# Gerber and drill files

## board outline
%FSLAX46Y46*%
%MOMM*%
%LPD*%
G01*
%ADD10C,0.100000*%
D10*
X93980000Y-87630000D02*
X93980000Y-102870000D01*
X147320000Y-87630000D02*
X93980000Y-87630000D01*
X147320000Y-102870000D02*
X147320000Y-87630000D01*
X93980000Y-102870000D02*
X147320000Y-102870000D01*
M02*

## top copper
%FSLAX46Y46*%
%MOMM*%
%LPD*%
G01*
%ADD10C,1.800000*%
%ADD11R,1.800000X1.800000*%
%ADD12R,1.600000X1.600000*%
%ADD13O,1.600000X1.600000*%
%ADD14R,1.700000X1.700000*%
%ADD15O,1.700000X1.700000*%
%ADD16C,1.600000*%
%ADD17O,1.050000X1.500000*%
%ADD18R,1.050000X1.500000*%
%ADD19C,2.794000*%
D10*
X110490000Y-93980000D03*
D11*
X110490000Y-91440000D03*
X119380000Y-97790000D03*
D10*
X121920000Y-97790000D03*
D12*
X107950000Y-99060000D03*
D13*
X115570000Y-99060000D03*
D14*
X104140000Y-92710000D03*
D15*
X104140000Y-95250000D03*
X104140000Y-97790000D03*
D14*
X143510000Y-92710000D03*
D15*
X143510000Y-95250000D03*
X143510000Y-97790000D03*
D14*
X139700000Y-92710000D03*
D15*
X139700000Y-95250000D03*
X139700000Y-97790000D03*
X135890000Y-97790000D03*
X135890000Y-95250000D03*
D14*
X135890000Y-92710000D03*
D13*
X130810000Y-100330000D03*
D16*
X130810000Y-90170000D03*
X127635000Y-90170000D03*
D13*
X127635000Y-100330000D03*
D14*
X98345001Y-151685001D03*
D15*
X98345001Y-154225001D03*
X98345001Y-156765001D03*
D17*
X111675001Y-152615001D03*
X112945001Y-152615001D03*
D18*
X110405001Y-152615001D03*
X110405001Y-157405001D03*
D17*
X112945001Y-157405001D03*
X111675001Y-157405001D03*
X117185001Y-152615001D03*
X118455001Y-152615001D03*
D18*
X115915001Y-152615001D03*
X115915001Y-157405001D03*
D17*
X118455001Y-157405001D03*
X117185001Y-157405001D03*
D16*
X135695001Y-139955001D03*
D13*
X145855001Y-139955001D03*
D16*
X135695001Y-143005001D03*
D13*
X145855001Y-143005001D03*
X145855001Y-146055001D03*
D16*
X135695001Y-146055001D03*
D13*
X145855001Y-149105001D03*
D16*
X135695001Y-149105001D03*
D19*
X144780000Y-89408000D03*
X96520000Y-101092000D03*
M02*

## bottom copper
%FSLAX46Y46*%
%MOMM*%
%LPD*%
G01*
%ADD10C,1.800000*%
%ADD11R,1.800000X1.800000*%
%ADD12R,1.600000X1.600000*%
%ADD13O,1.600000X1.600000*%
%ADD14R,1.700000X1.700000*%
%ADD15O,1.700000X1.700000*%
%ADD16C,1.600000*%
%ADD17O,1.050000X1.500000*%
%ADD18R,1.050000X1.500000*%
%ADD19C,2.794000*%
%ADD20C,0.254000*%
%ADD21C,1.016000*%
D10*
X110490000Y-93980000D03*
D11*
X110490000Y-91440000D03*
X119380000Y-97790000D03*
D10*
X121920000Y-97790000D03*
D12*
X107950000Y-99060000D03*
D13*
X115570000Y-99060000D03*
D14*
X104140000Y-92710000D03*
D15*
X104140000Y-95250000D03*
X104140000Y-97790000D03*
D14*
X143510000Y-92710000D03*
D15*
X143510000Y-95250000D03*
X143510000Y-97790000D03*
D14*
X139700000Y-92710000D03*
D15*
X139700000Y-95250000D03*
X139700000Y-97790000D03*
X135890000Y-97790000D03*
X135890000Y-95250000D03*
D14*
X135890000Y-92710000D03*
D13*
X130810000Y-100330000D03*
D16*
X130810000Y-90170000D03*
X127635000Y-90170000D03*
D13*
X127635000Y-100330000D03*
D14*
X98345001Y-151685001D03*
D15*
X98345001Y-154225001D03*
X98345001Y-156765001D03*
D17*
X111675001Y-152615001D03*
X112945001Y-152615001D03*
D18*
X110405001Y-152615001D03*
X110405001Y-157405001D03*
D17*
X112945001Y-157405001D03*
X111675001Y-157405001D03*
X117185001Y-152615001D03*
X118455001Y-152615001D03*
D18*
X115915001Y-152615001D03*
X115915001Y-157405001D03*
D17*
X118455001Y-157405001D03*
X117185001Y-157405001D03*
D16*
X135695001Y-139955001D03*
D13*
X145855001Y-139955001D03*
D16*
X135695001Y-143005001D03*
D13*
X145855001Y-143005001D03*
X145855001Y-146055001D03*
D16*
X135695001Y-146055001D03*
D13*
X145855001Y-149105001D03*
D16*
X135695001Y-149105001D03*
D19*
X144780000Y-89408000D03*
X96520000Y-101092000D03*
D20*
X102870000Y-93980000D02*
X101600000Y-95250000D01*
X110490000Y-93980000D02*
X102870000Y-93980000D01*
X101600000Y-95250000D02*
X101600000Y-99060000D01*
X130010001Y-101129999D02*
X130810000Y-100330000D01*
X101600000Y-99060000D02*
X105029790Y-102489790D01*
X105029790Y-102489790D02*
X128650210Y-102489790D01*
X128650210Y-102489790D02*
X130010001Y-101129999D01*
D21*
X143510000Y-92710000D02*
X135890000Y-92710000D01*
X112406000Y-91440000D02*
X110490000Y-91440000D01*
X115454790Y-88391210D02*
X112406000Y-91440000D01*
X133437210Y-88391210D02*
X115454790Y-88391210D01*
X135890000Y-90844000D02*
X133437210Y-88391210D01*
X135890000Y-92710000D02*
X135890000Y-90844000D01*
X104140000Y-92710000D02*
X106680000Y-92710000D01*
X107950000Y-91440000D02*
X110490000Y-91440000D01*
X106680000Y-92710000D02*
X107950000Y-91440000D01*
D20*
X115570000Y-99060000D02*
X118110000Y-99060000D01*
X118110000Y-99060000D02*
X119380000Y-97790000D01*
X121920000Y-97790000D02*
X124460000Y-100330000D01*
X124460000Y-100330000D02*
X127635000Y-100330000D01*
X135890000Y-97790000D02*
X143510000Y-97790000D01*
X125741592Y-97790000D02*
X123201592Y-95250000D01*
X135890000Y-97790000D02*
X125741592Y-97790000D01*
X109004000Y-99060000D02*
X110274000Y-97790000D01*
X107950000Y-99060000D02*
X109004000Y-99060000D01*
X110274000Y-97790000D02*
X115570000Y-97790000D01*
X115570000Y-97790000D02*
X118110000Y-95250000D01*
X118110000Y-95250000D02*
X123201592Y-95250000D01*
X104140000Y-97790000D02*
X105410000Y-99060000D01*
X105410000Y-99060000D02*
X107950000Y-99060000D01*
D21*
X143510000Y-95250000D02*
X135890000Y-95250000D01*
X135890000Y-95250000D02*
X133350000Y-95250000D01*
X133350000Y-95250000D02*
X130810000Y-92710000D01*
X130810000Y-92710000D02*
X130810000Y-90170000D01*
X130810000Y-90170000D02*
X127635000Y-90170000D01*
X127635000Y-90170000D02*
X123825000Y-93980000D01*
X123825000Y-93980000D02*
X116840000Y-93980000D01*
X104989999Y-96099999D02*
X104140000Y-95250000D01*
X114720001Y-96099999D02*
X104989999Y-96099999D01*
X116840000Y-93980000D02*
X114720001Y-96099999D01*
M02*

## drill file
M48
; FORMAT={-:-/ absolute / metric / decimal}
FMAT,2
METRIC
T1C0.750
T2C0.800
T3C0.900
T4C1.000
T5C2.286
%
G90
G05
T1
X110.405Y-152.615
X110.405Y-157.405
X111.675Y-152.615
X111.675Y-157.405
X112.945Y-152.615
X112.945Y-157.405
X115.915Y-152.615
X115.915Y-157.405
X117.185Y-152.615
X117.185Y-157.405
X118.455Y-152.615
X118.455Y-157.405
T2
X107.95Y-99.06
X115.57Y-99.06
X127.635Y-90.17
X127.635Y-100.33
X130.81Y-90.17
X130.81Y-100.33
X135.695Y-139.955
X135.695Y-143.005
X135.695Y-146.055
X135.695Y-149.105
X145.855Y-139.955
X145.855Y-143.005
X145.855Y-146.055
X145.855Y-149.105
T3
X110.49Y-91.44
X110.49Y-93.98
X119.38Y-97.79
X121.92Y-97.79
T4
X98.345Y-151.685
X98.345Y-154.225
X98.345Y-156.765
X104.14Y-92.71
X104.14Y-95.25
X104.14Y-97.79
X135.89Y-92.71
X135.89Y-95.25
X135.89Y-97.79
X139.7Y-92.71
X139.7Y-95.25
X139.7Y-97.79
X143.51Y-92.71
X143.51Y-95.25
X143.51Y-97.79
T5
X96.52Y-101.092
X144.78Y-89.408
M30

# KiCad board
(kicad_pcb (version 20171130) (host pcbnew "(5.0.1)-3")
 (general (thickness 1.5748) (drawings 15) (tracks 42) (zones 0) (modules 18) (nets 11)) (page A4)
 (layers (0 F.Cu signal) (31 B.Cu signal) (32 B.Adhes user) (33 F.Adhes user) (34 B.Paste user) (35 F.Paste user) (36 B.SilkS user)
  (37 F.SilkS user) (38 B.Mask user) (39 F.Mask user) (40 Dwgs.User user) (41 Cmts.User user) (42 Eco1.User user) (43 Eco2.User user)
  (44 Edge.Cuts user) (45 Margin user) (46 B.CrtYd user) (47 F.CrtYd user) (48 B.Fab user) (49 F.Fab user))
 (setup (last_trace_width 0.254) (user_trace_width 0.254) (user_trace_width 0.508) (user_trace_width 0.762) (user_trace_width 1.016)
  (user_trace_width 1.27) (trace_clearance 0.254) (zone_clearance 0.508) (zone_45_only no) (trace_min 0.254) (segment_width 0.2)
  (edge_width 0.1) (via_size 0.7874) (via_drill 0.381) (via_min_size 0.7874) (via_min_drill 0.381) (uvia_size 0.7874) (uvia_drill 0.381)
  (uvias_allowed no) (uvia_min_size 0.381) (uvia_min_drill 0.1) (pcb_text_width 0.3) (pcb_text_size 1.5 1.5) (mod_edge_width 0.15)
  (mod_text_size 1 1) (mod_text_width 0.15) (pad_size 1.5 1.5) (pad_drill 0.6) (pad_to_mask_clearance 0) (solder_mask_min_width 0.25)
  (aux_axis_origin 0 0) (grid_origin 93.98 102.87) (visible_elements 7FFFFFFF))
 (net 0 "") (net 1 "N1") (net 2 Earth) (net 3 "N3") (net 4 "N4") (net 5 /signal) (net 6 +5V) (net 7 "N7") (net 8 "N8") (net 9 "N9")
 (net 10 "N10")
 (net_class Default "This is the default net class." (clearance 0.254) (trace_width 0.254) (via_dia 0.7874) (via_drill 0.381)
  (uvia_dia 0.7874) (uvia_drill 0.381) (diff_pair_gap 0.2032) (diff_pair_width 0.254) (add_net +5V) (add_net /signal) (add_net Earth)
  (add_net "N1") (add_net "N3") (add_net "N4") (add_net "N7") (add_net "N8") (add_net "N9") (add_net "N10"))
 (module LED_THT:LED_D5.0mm (layer F.Cu) (at 110.49 91.44 270)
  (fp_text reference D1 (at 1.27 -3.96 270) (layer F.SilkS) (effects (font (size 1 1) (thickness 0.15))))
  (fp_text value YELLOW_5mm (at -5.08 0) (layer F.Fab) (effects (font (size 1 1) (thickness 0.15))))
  (pad 2 thru_hole circle (at 2.54 0 270) (size 1.8 1.8) (drill 0.9) (layers *.Cu *.Mask) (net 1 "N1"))
  (pad 1 thru_hole rect (at 0 0 270) (size 1.8 1.8) (drill 0.9) (layers *.Cu *.Mask) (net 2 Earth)))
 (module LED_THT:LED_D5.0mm (layer F.Cu) (at 119.38 97.79)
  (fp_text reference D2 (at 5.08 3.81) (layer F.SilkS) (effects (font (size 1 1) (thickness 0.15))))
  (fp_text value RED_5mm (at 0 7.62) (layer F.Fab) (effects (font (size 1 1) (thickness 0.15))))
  (pad 1 thru_hole rect (at 0 0) (size 1.8 1.8) (drill 0.9) (layers *.Cu *.Mask) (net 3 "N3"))
  (pad 2 thru_hole circle (at 2.54 0) (size 1.8 1.8) (drill 0.9) (layers *.Cu *.Mask) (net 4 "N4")))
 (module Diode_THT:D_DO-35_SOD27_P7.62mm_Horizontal (layer F.Cu) (at 107.95 99.06)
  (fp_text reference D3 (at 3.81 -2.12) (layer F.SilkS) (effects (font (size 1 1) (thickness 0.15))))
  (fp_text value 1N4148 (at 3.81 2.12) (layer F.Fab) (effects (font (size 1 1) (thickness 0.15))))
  (pad 1 thru_hole rect (at 0 0) (size 1.6 1.6) (drill 0.8) (layers *.Cu *.Mask) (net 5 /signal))
  (pad 2 thru_hole oval (at 7.62 0) (size 1.6 1.6) (drill 0.8) (layers *.Cu *.Mask) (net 3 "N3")))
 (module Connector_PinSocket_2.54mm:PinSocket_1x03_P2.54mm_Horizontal (layer F.Cu) (at 104.14 92.71)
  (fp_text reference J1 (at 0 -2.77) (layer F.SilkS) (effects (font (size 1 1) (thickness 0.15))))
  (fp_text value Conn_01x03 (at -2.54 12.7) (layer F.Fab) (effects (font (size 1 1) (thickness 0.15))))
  (pad 1 thru_hole rect (at 0 0) (size 1.7 1.7) (drill 1) (layers *.Cu *.Mask) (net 2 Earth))
  (pad 2 thru_hole oval (at 0 2.54) (size 1.7 1.7) (drill 1) (layers *.Cu *.Mask) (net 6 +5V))
  (pad 3 thru_hole oval (at 0 5.08) (size 1.7 1.7) (drill 1) (layers *.Cu *.Mask) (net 5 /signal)))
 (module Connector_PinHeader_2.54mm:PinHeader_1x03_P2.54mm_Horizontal (layer F.Cu) (at 143.51 92.71)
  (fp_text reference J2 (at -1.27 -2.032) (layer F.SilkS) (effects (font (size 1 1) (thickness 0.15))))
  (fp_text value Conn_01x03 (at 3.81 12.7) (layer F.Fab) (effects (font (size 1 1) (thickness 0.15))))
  (pad 1 thru_hole rect (at 0 0) (size 1.7 1.7) (drill 1) (layers *.Cu *.Mask) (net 2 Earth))
  (pad 2 thru_hole oval (at 0 2.54) (size 1.7 1.7) (drill 1) (layers *.Cu *.Mask) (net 6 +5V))
  (pad 3 thru_hole oval (at 0 5.08) (size 1.7 1.7) (drill 1) (layers *.Cu *.Mask) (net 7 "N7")))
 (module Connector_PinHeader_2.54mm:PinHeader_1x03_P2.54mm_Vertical (layer F.Cu) (at 139.7 92.71)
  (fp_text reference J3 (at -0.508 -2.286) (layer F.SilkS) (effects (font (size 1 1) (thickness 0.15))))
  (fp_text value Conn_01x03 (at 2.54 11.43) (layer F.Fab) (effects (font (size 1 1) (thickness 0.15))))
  (pad 1 thru_hole rect (at 0 0) (size 1.7 1.7) (drill 1) (layers *.Cu *.Mask) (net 2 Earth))
  (pad 2 thru_hole oval (at 0 2.54) (size 1.7 1.7) (drill 1) (layers *.Cu *.Mask) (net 6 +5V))
  (pad 3 thru_hole oval (at 0 5.08) (size 1.7 1.7) (drill 1) (layers *.Cu *.Mask) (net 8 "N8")))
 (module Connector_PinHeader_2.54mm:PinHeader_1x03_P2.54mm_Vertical (layer F.Cu) (at 135.89 92.71)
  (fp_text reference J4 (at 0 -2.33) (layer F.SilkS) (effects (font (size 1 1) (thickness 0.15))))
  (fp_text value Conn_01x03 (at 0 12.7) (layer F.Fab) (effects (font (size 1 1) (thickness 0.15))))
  (pad 3 thru_hole oval (at 0 5.08) (size 1.7 1.7) (drill 1) (layers *.Cu *.Mask) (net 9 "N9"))
  (pad 2 thru_hole oval (at 0 2.54) (size 1.7 1.7) (drill 1) (layers *.Cu *.Mask) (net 6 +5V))
  (pad 1 thru_hole rect (at 0 0) (size 1.7 1.7) (drill 1) (layers *.Cu *.Mask) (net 2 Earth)))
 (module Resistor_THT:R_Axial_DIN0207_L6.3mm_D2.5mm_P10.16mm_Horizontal (layer F.Cu) (at 130.81 90.17 270)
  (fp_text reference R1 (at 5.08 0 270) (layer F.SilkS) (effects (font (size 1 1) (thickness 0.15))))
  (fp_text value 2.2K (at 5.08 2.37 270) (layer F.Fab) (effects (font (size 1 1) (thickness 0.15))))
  (pad 2 thru_hole oval (at 10.16 0 270) (size 1.6 1.6) (drill 0.8) (layers *.Cu *.Mask) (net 1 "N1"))
  (pad 1 thru_hole circle (at 0 0 270) (size 1.6 1.6) (drill 0.8) (layers *.Cu *.Mask) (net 6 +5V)))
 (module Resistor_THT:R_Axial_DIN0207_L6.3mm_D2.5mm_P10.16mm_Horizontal (layer F.Cu) (at 127.635 90.17 270)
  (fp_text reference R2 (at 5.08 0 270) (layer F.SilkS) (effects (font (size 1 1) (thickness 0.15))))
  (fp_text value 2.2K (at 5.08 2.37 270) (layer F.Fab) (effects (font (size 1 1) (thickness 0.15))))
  (pad 1 thru_hole circle (at 0 0 270) (size 1.6 1.6) (drill 0.8) (layers *.Cu *.Mask) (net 6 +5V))
  (pad 2 thru_hole oval (at 10.16 0 270) (size 1.6 1.6) (drill 0.8) (layers *.Cu *.Mask) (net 4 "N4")))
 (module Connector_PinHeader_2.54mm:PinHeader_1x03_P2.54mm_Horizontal (layer F.Cu) (at 98.345001 151.685001)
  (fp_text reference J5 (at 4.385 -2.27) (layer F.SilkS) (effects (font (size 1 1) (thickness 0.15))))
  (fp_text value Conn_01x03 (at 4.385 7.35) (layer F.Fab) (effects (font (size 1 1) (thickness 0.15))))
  (pad 1 thru_hole rect (at 0 0) (size 1.7 1.7) (drill 1) (layers *.Cu *.Mask) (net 2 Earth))
  (pad 2 thru_hole oval (at 0 2.54) (size 1.7 1.7) (drill 1) (layers *.Cu *.Mask) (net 6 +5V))
  (pad 3 thru_hole oval (at 0 5.08) (size 1.7 1.7) (drill 1) (layers *.Cu *.Mask) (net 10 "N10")))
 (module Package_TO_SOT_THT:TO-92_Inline (layer F.Cu) (at 110.405001 152.615001)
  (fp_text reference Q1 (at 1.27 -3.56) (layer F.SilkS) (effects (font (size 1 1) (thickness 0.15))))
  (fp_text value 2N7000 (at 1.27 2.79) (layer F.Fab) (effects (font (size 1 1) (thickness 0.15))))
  (pad 2 thru_hole oval (at 1.27 0) (size 1.05 1.5) (drill 0.75) (layers *.Cu *.Mask) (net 7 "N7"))
  (pad 3 thru_hole oval (at 2.54 0) (size 1.05 1.5) (drill 0.75) (layers *.Cu *.Mask) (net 5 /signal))
  (pad 1 thru_hole rect (at 0 0) (size 1.05 1.5) (drill 0.75) (layers *.Cu *.Mask) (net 2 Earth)))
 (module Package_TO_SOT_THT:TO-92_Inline (layer F.Cu) (at 110.405001 157.405001)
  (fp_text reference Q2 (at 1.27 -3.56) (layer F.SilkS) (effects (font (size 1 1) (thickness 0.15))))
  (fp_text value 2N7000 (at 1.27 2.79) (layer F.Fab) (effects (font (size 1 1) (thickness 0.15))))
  (pad 1 thru_hole rect (at 0 0) (size 1.05 1.5) (drill 0.75) (layers *.Cu *.Mask) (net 2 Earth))
  (pad 3 thru_hole oval (at 2.54 0) (size 1.05 1.5) (drill 0.75) (layers *.Cu *.Mask) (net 5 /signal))
  (pad 2 thru_hole oval (at 1.27 0) (size 1.05 1.5) (drill 0.75) (layers *.Cu *.Mask) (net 8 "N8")))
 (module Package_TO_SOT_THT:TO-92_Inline (layer F.Cu) (at 115.915001 152.615001)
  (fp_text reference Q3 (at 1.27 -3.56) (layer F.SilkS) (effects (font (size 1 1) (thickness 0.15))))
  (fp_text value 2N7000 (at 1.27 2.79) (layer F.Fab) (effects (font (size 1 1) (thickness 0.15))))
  (pad 2 thru_hole oval (at 1.27 0) (size 1.05 1.5) (drill 0.75) (layers *.Cu *.Mask) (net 9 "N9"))
  (pad 3 thru_hole oval (at 2.54 0) (size 1.05 1.5) (drill 0.75) (layers *.Cu *.Mask) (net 5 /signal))
  (pad 1 thru_hole rect (at 0 0) (size 1.05 1.5) (drill 0.75) (layers *.Cu *.Mask) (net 2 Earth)))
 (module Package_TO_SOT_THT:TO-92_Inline (layer F.Cu) (at 115.915001 157.405001)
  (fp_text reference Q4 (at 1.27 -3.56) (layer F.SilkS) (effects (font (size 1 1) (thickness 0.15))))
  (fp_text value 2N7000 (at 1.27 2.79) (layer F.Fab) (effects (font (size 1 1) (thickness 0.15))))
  (pad 1 thru_hole rect (at 0 0) (size 1.05 1.5) (drill 0.75) (layers *.Cu *.Mask) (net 2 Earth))
  (pad 3 thru_hole oval (at 2.54 0) (size 1.05 1.5) (drill 0.75) (layers *.Cu *.Mask) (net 5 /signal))
  (pad 2 thru_hole oval (at 1.27 0) (size 1.05 1.5) (drill 0.75) (layers *.Cu *.Mask) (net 10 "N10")))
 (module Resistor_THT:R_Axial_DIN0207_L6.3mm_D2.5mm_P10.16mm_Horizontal (layer F.Cu) (at 135.695001 139.955001)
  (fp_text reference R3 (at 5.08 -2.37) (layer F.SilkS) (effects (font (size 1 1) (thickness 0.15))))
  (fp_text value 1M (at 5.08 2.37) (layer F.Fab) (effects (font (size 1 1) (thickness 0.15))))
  (pad 1 thru_hole circle (at 0 0) (size 1.6 1.6) (drill 0.8) (layers *.Cu *.Mask) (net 7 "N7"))
  (pad 2 thru_hole oval (at 10.16 0) (size 1.6 1.6) (drill 0.8) (layers *.Cu *.Mask) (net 2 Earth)))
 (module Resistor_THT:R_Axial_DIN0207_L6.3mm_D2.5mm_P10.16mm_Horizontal (layer F.Cu) (at 135.695001 143.005001)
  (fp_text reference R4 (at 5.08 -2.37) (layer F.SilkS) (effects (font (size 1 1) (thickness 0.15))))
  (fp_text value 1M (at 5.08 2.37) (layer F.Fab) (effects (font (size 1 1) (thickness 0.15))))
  (pad 1 thru_hole circle (at 0 0) (size 1.6 1.6) (drill 0.8) (layers *.Cu *.Mask) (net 8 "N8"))
  (pad 2 thru_hole oval (at 10.16 0) (size 1.6 1.6) (drill 0.8) (layers *.Cu *.Mask) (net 2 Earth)))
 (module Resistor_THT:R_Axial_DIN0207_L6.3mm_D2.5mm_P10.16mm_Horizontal (layer F.Cu) (at 135.695001 146.055001)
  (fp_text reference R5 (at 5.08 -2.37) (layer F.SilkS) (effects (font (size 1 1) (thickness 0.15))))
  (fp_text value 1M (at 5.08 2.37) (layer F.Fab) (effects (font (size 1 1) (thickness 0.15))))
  (pad 2 thru_hole oval (at 10.16 0) (size 1.6 1.6) (drill 0.8) (layers *.Cu *.Mask) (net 2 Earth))
  (pad 1 thru_hole circle (at 0 0) (size 1.6 1.6) (drill 0.8) (layers *.Cu *.Mask) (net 9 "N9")))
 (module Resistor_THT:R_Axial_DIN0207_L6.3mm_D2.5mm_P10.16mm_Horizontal (layer F.Cu) (at 135.695001 149.105001)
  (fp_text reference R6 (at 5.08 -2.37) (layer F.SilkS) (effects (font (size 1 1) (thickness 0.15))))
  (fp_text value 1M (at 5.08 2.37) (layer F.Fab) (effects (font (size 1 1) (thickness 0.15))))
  (pad 2 thru_hole oval (at 10.16 0) (size 1.6 1.6) (drill 0.8) (layers *.Cu *.Mask) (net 2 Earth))
  (pad 1 thru_hole circle (at 0 0) (size 1.6 1.6) (drill 0.8) (layers *.Cu *.Mask) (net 10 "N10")))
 (gr_line (start 93.98 87.63) (end 93.98 102.87) (layer Edge.Cuts) (width 0.1))
 (gr_line (start 147.32 87.63) (end 93.98 87.63) (layer Edge.Cuts) (width 0.1))
 (gr_line (start 147.32 102.87) (end 147.32 87.63) (layer Edge.Cuts) (width 0.1))
 (gr_line (start 93.98 102.87) (end 147.32 102.87) (layer Edge.Cuts) (width 0.1))
 (via (at 144.78 89.408) (size 2.794) (drill 2.286) (layers F.Cu B.Cu) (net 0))
 (via (at 96.52 101.092) (size 2.794) (drill 2.286) (layers F.Cu B.Cu) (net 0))
 (segment (start 102.87 93.98) (end 101.6 95.25) (width 0.254) (layer B.Cu) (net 1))
 (segment (start 110.49 93.98) (end 102.87 93.98) (width 0.254) (layer B.Cu) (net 1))
 (segment (start 101.6 95.25) (end 101.6 99.06) (width 0.254) (layer B.Cu) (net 1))
 (segment (start 130.010001 101.129999) (end 130.81 100.33) (width 0.254) (layer B.Cu) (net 1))
 (segment (start 101.6 99.06) (end 105.02979 102.48979) (width 0.254) (layer B.Cu) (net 1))
 (segment (start 105.02979 102.48979) (end 128.65021 102.48979) (width 0.254) (layer B.Cu) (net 1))
 (segment (start 128.65021 102.48979) (end 130.010001 101.129999) (width 0.254) (layer B.Cu) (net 1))
 (segment (start 143.51 92.71) (end 135.89 92.71) (width 1.016) (layer B.Cu) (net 2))
 (segment (start 112.406 91.44) (end 110.49 91.44) (width 1.016) (layer B.Cu) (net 2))
 (segment (start 115.45479 88.39121) (end 112.406 91.44) (width 1.016) (layer B.Cu) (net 2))
 (segment (start 133.43721 88.39121) (end 115.45479 88.39121) (width 1.016) (layer B.Cu) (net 2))
 (segment (start 135.89 90.844) (end 133.43721 88.39121) (width 1.016) (layer B.Cu) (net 2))
 (segment (start 135.89 92.71) (end 135.89 90.844) (width 1.016) (layer B.Cu) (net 2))
 (segment (start 104.14 92.71) (end 106.68 92.71) (width 1.016) (layer B.Cu) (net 2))
 (segment (start 107.95 91.44) (end 110.49 91.44) (width 1.016) (layer B.Cu) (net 2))
 (segment (start 106.68 92.71) (end 107.95 91.44) (width 1.016) (layer B.Cu) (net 2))
 (segment (start 115.57 99.06) (end 118.11 99.06) (width 0.254) (layer B.Cu) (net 3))
 (segment (start 118.11 99.06) (end 119.38 97.79) (width 0.254) (layer B.Cu) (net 3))
 (segment (start 121.92 97.79) (end 124.46 100.33) (width 0.254) (layer B.Cu) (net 4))
 (segment (start 124.46 100.33) (end 127.635 100.33) (width 0.254) (layer B.Cu) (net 4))
 (segment (start 135.89 97.79) (end 143.51 97.79) (width 0.254) (layer B.Cu) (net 5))
 (segment (start 125.741592 97.79) (end 123.201592 95.25) (width 0.254) (layer B.Cu) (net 5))
 (segment (start 135.89 97.79) (end 125.741592 97.79) (width 0.254) (layer B.Cu) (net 5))
 (segment (start 109.004 99.06) (end 110.274 97.79) (width 0.254) (layer B.Cu) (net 5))
 (segment (start 107.95 99.06) (end 109.004 99.06) (width 0.254) (layer B.Cu) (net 5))
 (segment (start 110.274 97.79) (end 115.57 97.79) (width 0.254) (layer B.Cu) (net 5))
 (segment (start 115.57 97.79) (end 118.11 95.25) (width 0.254) (layer B.Cu) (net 5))
 (segment (start 118.11 95.25) (end 123.201592 95.25) (width 0.254) (layer B.Cu) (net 5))
 (segment (start 104.14 97.79) (end 105.41 99.06) (width 0.254) (layer B.Cu) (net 5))
 (segment (start 105.41 99.06) (end 107.95 99.06) (width 0.254) (layer B.Cu) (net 5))
 (segment (start 143.51 95.25) (end 135.89 95.25) (width 1.016) (layer B.Cu) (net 6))
 (segment (start 135.89 95.25) (end 133.35 95.25) (width 1.016) (layer B.Cu) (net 6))
 (segment (start 133.35 95.25) (end 130.81 92.71) (width 1.016) (layer B.Cu) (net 6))
 (segment (start 130.81 92.71) (end 130.81 90.17) (width 1.016) (layer B.Cu) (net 6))
 (segment (start 130.81 90.17) (end 127.635 90.17) (width 1.016) (layer B.Cu) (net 6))
 (segment (start 127.635 90.17) (end 123.825 93.98) (width 1.016) (layer B.Cu) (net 6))
 (segment (start 123.825 93.98) (end 116.84 93.98) (width 1.016) (layer B.Cu) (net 6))
 (segment (start 104.989999 96.099999) (end 104.14 95.25) (width 1.016) (layer B.Cu) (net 6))
 (segment (start 114.720001 96.099999) (end 104.989999 96.099999) (width 1.016) (layer B.Cu) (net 6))
 (segment (start 116.84 93.98) (end 114.720001 96.099999) (width 1.016) (layer B.Cu) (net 6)))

